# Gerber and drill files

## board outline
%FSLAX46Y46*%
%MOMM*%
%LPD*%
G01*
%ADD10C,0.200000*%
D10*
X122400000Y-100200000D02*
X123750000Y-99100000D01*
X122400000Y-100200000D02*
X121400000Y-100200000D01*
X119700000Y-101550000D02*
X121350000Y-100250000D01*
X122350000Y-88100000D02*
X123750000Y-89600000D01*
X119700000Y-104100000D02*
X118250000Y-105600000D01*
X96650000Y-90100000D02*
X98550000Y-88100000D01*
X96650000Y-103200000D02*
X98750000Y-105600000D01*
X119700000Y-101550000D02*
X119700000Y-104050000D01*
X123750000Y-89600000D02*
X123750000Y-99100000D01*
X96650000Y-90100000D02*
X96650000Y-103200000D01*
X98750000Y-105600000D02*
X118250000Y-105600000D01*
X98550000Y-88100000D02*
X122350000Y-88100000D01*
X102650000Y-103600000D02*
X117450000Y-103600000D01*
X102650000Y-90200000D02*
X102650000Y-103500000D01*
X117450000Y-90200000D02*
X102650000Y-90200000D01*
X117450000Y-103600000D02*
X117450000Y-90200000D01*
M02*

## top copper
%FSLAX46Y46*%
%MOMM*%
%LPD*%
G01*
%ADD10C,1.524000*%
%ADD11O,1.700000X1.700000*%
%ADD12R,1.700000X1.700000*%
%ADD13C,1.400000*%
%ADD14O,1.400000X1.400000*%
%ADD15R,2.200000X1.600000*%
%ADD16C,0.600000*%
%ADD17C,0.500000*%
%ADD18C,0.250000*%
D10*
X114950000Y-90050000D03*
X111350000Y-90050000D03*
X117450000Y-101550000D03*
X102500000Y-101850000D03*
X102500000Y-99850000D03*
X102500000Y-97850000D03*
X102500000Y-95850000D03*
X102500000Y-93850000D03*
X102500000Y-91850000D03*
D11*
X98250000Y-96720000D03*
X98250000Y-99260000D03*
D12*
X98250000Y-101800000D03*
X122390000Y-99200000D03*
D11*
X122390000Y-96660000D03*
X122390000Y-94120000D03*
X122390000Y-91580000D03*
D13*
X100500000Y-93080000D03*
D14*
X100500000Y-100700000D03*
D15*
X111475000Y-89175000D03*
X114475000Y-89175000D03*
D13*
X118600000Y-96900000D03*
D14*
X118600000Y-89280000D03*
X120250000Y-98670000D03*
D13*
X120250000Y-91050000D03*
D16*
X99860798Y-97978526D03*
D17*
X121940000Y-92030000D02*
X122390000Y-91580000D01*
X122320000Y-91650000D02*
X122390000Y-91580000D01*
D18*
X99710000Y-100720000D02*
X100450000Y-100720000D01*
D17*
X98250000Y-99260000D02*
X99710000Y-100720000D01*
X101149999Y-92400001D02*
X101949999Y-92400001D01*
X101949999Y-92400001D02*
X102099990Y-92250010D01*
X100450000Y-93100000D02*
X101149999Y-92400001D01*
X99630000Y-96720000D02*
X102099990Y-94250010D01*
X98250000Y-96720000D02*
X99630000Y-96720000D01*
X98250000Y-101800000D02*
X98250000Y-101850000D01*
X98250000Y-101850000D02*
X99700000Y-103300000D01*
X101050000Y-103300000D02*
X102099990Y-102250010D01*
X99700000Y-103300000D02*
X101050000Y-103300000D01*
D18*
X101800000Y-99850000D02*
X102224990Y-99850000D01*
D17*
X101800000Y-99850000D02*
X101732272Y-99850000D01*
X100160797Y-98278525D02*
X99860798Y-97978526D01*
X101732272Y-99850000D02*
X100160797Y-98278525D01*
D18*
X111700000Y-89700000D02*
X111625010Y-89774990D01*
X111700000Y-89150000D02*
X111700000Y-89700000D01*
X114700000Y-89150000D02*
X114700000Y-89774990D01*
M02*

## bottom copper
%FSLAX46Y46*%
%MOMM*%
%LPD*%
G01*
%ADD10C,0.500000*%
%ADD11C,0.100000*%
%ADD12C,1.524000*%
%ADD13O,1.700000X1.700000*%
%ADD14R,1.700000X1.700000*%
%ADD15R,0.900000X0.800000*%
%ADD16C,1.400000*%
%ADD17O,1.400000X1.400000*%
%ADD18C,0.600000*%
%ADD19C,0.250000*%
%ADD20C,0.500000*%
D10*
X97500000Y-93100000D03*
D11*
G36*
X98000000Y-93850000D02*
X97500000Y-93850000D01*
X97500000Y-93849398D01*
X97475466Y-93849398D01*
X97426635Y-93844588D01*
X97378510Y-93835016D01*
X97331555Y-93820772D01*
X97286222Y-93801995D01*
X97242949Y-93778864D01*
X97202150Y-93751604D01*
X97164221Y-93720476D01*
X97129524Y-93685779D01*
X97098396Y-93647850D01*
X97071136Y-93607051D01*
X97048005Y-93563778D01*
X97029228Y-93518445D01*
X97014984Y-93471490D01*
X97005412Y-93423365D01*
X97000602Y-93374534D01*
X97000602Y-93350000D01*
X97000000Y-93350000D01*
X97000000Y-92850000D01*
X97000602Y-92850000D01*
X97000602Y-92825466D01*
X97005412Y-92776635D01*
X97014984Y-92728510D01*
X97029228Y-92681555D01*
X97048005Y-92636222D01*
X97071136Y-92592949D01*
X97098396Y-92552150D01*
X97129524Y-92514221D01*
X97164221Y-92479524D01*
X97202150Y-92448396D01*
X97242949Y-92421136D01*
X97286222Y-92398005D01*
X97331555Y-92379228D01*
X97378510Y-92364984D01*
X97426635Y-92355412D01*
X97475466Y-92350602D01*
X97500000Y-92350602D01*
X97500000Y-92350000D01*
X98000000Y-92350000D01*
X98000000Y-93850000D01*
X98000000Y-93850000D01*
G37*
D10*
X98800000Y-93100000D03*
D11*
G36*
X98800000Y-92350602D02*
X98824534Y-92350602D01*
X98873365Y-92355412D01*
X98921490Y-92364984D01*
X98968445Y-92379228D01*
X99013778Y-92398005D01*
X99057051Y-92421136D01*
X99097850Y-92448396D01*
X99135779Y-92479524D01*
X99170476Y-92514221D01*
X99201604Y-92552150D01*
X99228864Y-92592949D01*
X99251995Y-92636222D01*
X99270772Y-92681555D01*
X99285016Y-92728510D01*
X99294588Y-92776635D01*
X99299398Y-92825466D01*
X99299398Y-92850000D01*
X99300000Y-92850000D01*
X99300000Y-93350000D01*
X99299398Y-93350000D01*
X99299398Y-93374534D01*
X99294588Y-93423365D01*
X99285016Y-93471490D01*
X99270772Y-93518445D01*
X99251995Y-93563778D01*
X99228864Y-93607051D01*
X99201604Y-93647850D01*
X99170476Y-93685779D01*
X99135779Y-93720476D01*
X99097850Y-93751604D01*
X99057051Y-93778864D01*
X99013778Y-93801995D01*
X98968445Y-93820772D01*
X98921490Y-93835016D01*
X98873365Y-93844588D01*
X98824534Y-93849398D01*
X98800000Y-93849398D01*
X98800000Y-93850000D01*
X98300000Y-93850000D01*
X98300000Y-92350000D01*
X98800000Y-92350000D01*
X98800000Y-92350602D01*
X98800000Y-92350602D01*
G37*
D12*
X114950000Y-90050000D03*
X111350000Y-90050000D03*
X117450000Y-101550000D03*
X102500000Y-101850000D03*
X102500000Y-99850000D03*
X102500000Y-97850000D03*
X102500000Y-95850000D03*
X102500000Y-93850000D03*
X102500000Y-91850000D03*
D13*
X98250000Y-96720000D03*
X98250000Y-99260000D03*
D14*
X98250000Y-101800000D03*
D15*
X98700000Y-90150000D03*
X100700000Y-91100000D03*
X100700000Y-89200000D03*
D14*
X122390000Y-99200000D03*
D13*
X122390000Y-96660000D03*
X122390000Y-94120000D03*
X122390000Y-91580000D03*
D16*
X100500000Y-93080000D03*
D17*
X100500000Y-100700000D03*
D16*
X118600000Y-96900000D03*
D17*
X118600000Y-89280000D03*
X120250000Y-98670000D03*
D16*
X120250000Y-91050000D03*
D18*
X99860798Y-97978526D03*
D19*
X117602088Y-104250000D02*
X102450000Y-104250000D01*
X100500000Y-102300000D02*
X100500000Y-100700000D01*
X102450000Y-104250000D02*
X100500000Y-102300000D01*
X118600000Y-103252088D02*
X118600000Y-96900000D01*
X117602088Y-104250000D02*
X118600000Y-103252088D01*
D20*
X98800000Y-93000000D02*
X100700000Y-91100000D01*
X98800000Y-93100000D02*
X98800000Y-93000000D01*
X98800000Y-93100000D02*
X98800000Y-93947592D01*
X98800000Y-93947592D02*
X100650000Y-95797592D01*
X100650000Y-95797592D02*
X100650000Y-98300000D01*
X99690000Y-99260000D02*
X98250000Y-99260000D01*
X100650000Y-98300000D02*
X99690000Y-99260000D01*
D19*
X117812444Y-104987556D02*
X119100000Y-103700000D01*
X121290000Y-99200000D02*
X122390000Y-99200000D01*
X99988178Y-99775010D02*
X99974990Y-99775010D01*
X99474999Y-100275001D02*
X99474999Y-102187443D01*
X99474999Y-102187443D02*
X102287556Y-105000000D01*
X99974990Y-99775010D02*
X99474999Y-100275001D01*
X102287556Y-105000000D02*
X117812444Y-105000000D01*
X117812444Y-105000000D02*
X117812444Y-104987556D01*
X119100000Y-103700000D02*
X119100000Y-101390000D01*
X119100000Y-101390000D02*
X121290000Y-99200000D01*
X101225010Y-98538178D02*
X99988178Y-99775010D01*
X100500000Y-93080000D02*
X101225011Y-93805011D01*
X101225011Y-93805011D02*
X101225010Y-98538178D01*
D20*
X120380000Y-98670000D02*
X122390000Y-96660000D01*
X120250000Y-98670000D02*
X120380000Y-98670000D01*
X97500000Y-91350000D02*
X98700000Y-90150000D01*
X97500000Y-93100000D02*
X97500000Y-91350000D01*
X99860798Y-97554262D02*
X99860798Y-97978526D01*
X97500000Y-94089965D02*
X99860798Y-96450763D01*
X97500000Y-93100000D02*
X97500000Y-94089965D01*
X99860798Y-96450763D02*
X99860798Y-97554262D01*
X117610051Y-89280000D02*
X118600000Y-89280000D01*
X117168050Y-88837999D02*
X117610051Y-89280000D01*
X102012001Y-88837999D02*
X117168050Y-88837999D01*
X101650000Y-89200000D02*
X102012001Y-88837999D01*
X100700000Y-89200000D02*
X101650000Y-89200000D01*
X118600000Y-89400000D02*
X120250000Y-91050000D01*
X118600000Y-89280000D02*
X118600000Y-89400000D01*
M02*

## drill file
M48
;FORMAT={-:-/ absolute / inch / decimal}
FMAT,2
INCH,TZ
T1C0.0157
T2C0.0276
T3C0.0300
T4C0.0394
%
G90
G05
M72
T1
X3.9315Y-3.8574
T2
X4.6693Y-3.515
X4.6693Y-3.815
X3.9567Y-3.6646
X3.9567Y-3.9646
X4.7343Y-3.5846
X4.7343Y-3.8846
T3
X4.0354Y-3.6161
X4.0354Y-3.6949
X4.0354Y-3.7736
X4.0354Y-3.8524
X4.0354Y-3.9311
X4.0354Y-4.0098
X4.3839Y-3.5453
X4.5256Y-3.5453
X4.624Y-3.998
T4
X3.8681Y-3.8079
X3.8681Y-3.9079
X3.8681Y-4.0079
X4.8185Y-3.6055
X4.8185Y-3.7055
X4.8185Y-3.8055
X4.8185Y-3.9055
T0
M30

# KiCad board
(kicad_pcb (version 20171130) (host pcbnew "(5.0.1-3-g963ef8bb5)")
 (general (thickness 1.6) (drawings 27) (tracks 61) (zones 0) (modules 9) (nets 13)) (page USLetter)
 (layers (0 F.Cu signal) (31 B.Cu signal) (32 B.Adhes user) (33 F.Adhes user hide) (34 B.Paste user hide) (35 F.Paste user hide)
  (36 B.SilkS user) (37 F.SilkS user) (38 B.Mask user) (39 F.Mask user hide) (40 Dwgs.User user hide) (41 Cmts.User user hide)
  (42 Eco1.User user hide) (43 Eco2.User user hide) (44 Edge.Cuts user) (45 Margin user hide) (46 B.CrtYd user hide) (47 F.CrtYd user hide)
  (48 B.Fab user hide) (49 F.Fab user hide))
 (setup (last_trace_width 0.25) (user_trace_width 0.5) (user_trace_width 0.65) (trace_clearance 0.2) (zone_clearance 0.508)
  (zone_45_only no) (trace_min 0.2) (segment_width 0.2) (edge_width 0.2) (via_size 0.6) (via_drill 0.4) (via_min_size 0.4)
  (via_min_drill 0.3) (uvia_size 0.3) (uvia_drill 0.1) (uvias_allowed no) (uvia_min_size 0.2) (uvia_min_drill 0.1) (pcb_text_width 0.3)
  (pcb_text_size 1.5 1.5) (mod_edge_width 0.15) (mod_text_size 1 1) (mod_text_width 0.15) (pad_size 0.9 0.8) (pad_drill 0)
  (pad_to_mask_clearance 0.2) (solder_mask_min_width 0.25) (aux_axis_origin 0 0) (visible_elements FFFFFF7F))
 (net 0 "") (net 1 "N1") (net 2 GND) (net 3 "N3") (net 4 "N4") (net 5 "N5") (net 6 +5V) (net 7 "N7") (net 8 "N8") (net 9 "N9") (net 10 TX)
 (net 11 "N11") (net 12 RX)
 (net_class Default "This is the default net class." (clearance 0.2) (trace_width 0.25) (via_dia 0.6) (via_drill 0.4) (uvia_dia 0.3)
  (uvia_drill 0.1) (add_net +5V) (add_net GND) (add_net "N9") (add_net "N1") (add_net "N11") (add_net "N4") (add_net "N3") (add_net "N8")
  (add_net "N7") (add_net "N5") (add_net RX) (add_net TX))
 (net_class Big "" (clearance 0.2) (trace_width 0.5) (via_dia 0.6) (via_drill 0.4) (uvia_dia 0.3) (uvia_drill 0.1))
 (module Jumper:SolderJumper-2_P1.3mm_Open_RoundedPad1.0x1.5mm (layer B.Cu) (at 98.15 93.1)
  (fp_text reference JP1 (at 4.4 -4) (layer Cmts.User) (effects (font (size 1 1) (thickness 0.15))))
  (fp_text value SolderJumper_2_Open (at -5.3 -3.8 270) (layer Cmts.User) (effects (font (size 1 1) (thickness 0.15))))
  (pad 1 smd custom (at -0.65 0) (size 1 0.5) (layers B.Cu B.Mask) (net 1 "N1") (zone_connect 0) (options (clearance outline) (anchor rect))
   (primitives))
  (pad 2 smd custom (at 0.65 0) (size 1 0.5) (layers B.Cu B.Mask) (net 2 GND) (zone_connect 0) (options (clearance outline) (anchor rect))
   (primitives)))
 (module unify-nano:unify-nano (layer F.Cu) (at 102.75 103.35)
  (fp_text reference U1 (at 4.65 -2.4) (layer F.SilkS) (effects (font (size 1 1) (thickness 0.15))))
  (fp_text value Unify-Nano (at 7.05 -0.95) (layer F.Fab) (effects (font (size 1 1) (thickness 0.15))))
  (pad 9 thru_hole circle (at 12.2 -13.3) (size 1.524 1.524) (drill 0.762) (layers *.Cu *.Mask) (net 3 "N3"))
  (pad 10 thru_hole circle (at 8.6 -13.3) (size 1.524 1.524) (drill 0.762) (layers *.Cu *.Mask) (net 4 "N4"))
  (pad 7 thru_hole circle (at 14.7 -1.8) (size 1.524 1.524) (drill 0.762) (layers *.Cu *.Mask) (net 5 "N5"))
  (pad 6 thru_hole circle (at -0.25 -1.5) (size 1.524 1.524) (drill 0.762) (layers *.Cu *.Mask) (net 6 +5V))
  (pad 5 thru_hole circle (at -0.25 -3.5) (size 1.524 1.524) (drill 0.762) (layers *.Cu *.Mask) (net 1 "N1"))
  (pad 4 thru_hole circle (at -0.25 -5.5) (size 1.524 1.524) (drill 0.762) (layers *.Cu *.Mask) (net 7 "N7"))
  (pad 3 thru_hole circle (at -0.25 -7.5) (size 1.524 1.524) (drill 0.762) (layers *.Cu *.Mask) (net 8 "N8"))
  (pad 2 thru_hole circle (at -0.25 -9.5) (size 1.524 1.524) (drill 0.762) (layers *.Cu *.Mask) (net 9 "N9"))
  (pad 1 thru_hole circle (at -0.25 -11.5) (size 1.524 1.524) (drill 0.762) (layers *.Cu *.Mask) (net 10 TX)))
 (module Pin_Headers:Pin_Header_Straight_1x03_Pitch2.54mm (layer F.Cu) (at 98.25 101.8 180)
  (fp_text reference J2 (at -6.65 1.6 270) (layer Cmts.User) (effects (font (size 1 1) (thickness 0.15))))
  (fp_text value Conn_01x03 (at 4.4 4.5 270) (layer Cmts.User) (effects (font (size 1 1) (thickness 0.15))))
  (pad 3 thru_hole oval (at 0 5.08 180) (size 1.7 1.7) (drill 1) (layers *.Cu *.Mask) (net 9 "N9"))
  (pad 2 thru_hole oval (at 0 2.54 180) (size 1.7 1.7) (drill 1) (layers *.Cu *.Mask) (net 2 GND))
  (pad 1 thru_hole rect (at 0 0 180) (size 1.7 1.7) (drill 1) (layers *.Cu *.Mask) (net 6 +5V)))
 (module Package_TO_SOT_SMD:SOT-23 (layer B.Cu) (at 99.7 90.15 180)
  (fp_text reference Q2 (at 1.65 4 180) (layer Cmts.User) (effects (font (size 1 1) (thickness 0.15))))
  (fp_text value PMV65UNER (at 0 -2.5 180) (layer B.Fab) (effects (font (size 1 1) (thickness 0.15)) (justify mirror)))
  (pad 3 smd rect (at 1 0 180) (size 0.9 0.8) (layers B.Cu B.Paste B.Mask) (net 1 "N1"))
  (pad 2 smd rect (at -1 -0.95 180) (size 0.9 0.8) (layers B.Cu B.Paste B.Mask) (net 2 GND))
  (pad 1 smd rect (at -1 0.95 180) (size 0.9 0.8) (layers B.Cu B.Paste B.Mask) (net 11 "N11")))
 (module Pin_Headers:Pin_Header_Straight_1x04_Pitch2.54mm (layer F.Cu) (at 122.39 99.2 180)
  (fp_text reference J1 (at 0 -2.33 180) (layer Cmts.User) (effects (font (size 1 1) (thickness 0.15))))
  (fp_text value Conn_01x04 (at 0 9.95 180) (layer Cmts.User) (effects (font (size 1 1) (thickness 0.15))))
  (pad 1 thru_hole rect (at 0 0 180) (size 1.7 1.7) (drill 1) (layers *.Cu *.Mask) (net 10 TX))
  (pad 2 thru_hole oval (at 0 2.54 180) (size 1.7 1.7) (drill 1) (layers *.Cu *.Mask) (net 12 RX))
  (pad 3 thru_hole oval (at 0 5.08 180) (size 1.7 1.7) (drill 1) (layers *.Cu *.Mask) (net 6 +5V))
  (pad 4 thru_hole oval (at 0 7.62 180) (size 1.7 1.7) (drill 1) (layers *.Cu *.Mask) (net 2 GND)))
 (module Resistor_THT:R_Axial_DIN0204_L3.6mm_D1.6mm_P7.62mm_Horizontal (layer F.Cu) (at 100.5 93.08 270)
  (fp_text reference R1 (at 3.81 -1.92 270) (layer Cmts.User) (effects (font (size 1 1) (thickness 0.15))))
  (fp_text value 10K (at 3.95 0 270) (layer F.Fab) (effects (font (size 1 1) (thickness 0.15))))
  (pad 1 thru_hole circle (at 0 0 270) (size 1.4 1.4) (drill 0.7) (layers *.Cu *.Mask) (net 10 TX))
  (pad 2 thru_hole oval (at 7.62 0 270) (size 1.4 1.4) (drill 0.7) (layers *.Cu *.Mask) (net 2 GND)))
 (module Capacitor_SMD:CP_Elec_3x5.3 (layer F.Cu) (at 112.975 89.175)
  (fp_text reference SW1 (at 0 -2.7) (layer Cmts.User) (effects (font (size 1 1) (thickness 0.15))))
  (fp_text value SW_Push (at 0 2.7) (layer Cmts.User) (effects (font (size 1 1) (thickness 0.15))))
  (pad 1 smd rect (at -1.5 0) (size 2.2 1.6) (layers F.Cu F.Paste F.Mask) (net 4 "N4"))
  (pad 2 smd rect (at 1.5 0) (size 2.2 1.6) (layers F.Cu F.Paste F.Mask) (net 3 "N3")))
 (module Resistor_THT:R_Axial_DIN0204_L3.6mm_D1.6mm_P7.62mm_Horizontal (layer F.Cu) (at 118.6 96.9 90)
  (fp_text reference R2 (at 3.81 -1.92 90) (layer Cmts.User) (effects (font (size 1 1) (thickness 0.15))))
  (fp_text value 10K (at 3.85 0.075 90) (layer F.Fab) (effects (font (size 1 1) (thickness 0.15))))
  (pad 1 thru_hole circle (at 0 0 90) (size 1.4 1.4) (drill 0.7) (layers *.Cu *.Mask) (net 2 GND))
  (pad 2 thru_hole oval (at 7.62 0 90) (size 1.4 1.4) (drill 0.7) (layers *.Cu *.Mask) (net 11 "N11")))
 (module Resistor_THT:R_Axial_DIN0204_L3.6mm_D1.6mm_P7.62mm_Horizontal (layer F.Cu) (at 120.25 91.05 270)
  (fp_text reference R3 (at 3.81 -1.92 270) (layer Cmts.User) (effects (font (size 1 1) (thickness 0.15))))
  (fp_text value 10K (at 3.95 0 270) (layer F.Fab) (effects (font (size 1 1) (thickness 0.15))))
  (pad 2 thru_hole oval (at 7.62 0 270) (size 1.4 1.4) (drill 0.7) (layers *.Cu *.Mask) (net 12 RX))
  (pad 1 thru_hole circle (at 0 0 270) (size 1.4 1.4) (drill 0.7) (layers *.Cu *.Mask) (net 11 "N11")))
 (gr_line (start 122.4 100.2) (end 123.75 99.1) (layer Edge.Cuts) (width 0.2))
 (gr_line (start 122.4 100.2) (end 121.4 100.2) (layer Edge.Cuts) (width 0.2))
 (gr_line (start 119.7 101.55) (end 121.35 100.25) (layer Edge.Cuts) (width 0.2))
 (gr_line (start 122.35 88.1) (end 123.75 89.6) (layer Edge.Cuts) (width 0.2))
 (gr_line (start 119.7 104.1) (end 118.25 105.6) (layer Edge.Cuts) (width 0.2))
 (gr_line (start 96.65 90.1) (end 98.55 88.1) (layer Edge.Cuts) (width 0.2))
 (gr_line (start 96.65 103.2) (end 98.75 105.6) (layer Edge.Cuts) (width 0.2))
 (gr_line (start 119.7 101.55) (end 119.7 104.05) (layer Edge.Cuts) (width 0.2))
 (gr_line (start 123.75 89.6) (end 123.75 99.1) (layer Edge.Cuts) (width 0.2))
 (gr_line (start 96.65 90.1) (end 96.65 103.2) (layer Edge.Cuts) (width 0.2))
 (gr_line (start 98.75 105.6) (end 118.25 105.6) (layer Edge.Cuts) (width 0.2))
 (gr_line (start 98.55 88.1) (end 122.35 88.1) (layer Edge.Cuts) (width 0.2))
 (gr_line (start 102.65 103.6) (end 117.45 103.6) (layer Edge.Cuts) (width 0.2))
 (gr_line (start 102.65 90.2) (end 102.65 103.5) (layer Edge.Cuts) (width 0.2))
 (gr_line (start 117.45 90.2) (end 102.65 90.2) (layer Edge.Cuts) (width 0.2))
 (gr_line (start 117.45 103.6) (end 117.45 90.2) (layer Edge.Cuts) (width 0.2))
 (segment (start 121.94 92.03) (end 122.39 91.58) (width 0.5) (layer F.Cu) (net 2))
 (segment (start 122.32 91.65) (end 122.39 91.58) (width 0.5) (layer F.Cu) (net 2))
 (segment (start 99.71 100.72) (end 100.45 100.72) (width 0.25) (layer F.Cu) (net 2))
 (segment (start 98.25 99.26) (end 99.71 100.72) (width 0.5) (layer F.Cu) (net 2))
 (segment (start 117.602088 104.25) (end 102.45 104.25) (width 0.25) (layer B.Cu) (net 2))
 (segment (start 100.5 102.3) (end 100.5 100.7) (width 0.25) (layer B.Cu) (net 2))
 (segment (start 102.45 104.25) (end 100.5 102.3) (width 0.25) (layer B.Cu) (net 2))
 (segment (start 118.6 103.252088) (end 118.6 96.9) (width 0.25) (layer B.Cu) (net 2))
 (segment (start 117.602088 104.25) (end 118.6 103.252088) (width 0.25) (layer B.Cu) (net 2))
 (segment (start 98.8 93) (end 100.7 91.1) (width 0.5) (layer B.Cu) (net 2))
 (segment (start 98.8 93.1) (end 98.8 93) (width 0.5) (layer B.Cu) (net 2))
 (segment (start 98.8 93.1) (end 98.8 93.947592) (width 0.5) (layer B.Cu) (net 2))
 (segment (start 98.8 93.947592) (end 100.65 95.797592) (width 0.5) (layer B.Cu) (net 2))
 (segment (start 100.65 95.797592) (end 100.65 98.3) (width 0.5) (layer B.Cu) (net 2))
 (segment (start 99.69 99.26) (end 98.25 99.26) (width 0.5) (layer B.Cu) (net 2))
 (segment (start 100.65 98.3) (end 99.69 99.26) (width 0.5) (layer B.Cu) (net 2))
 (segment (start 101.149999 92.400001) (end 101.949999 92.400001) (width 0.5) (layer F.Cu) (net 10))
 (segment (start 101.949999 92.400001) (end 102.09999 92.25001) (width 0.5) (layer F.Cu) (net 10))
 (segment (start 100.45 93.1) (end 101.149999 92.400001) (width 0.5) (layer F.Cu) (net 10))
 (segment (start 117.812444 104.987556) (end 119.1 103.7) (width 0.25) (layer B.Cu) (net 10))
 (segment (start 121.29 99.2) (end 122.39 99.2) (width 0.25) (layer B.Cu) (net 10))
 (segment (start 99.988178 99.77501) (end 99.97499 99.77501) (width 0.25) (layer B.Cu) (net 10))
 (segment (start 99.474999 100.275001) (end 99.474999 102.187443) (width 0.25) (layer B.Cu) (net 10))
 (segment (start 99.474999 102.187443) (end 102.287556 105) (width 0.25) (layer B.Cu) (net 10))
 (segment (start 99.97499 99.77501) (end 99.474999 100.275001) (width 0.25) (layer B.Cu) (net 10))
 (segment (start 102.287556 105) (end 117.812444 105) (width 0.25) (layer B.Cu) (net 10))
 (segment (start 117.812444 105) (end 117.812444 104.987556) (width 0.25) (layer B.Cu) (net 10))
 (segment (start 119.1 103.7) (end 119.1 101.39) (width 0.25) (layer B.Cu) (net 10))
 (segment (start 119.1 101.39) (end 121.29 99.2) (width 0.25) (layer B.Cu) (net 10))
 (segment (start 101.22501 98.538178) (end 99.988178 99.77501) (width 0.25) (layer B.Cu) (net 10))
 (segment (start 100.5 93.08) (end 101.225011 93.805011) (width 0.25) (layer B.Cu) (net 10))
 (segment (start 101.225011 93.805011) (end 101.22501 98.538178) (width 0.25) (layer B.Cu) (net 10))
 (segment (start 99.63 96.72) (end 102.09999 94.25001) (width 0.5) (layer F.Cu) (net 9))
 (segment (start 98.25 96.72) (end 99.63 96.72) (width 0.5) (layer F.Cu) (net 9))
 (segment (start 120.38 98.67) (end 122.39 96.66) (width 0.5) (layer B.Cu) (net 12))
 (segment (start 120.25 98.67) (end 120.38 98.67) (width 0.5) (layer B.Cu) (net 12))
 (segment (start 98.25 101.8) (end 98.25 101.85) (width 0.5) (layer F.Cu) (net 6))
 (segment (start 98.25 101.85) (end 99.7 103.3) (width 0.5) (layer F.Cu) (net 6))
 (segment (start 101.05 103.3) (end 102.09999 102.25001) (width 0.5) (layer F.Cu) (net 6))
 (segment (start 99.7 103.3) (end 101.05 103.3) (width 0.5) (layer F.Cu) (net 6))
 (segment (start 101.8 99.85) (end 102.22499 99.85) (width 0.25) (layer F.Cu) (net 1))
 (segment (start 97.5 91.35) (end 98.7 90.15) (width 0.5) (layer B.Cu) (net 1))
 (segment (start 97.5 93.1) (end 97.5 91.35) (width 0.5) (layer B.Cu) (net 1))
 (segment (start 99.860798 97.554262) (end 99.860798 97.978526) (width 0.5) (layer B.Cu) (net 1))
 (segment (start 97.5 94.089965) (end 99.860798 96.450763) (width 0.5) (layer B.Cu) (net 1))
 (segment (start 101.8 99.85) (end 101.732272 99.85) (width 0.5) (layer F.Cu) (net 1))
 (via (at 99.860798 97.978526) (size 0.6) (drill 0.4) (layers F.Cu B.Cu) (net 1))
 (segment (start 97.5 93.1) (end 97.5 94.089965) (width 0.5) (layer B.Cu) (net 1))
 (segment (start 100.160797 98.278525) (end 99.860798 97.978526) (width 0.5) (layer F.Cu) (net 1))
 (segment (start 101.732272 99.85) (end 100.160797 98.278525) (width 0.5) (layer F.Cu) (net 1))
 (segment (start 99.860798 96.450763) (end 99.860798 97.554262) (width 0.5) (layer B.Cu) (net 1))
 (segment (start 117.610051 89.28) (end 118.6 89.28) (width 0.5) (layer B.Cu) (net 11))
 (segment (start 117.16805 88.837999) (end 117.610051 89.28) (width 0.5) (layer B.Cu) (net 11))
 (segment (start 102.012001 88.837999) (end 117.16805 88.837999) (width 0.5) (layer B.Cu) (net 11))
 (segment (start 101.65 89.2) (end 102.012001 88.837999) (width 0.5) (layer B.Cu) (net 11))
 (segment (start 100.7 89.2) (end 101.65 89.2) (width 0.5) (layer B.Cu) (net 11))
 (segment (start 118.6 89.4) (end 120.25 91.05) (width 0.5) (layer B.Cu) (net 11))
 (segment (start 118.6 89.28) (end 118.6 89.4) (width 0.5) (layer B.Cu) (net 11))
 (segment (start 111.7 89.7) (end 111.62501 89.77499) (width 0.25) (layer F.Cu) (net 4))
 (segment (start 111.7 89.15) (end 111.7 89.7) (width 0.25) (layer F.Cu) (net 4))
 (segment (start 114.7 89.15) (end 114.7 89.77499) (width 0.25) (layer F.Cu) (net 3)))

